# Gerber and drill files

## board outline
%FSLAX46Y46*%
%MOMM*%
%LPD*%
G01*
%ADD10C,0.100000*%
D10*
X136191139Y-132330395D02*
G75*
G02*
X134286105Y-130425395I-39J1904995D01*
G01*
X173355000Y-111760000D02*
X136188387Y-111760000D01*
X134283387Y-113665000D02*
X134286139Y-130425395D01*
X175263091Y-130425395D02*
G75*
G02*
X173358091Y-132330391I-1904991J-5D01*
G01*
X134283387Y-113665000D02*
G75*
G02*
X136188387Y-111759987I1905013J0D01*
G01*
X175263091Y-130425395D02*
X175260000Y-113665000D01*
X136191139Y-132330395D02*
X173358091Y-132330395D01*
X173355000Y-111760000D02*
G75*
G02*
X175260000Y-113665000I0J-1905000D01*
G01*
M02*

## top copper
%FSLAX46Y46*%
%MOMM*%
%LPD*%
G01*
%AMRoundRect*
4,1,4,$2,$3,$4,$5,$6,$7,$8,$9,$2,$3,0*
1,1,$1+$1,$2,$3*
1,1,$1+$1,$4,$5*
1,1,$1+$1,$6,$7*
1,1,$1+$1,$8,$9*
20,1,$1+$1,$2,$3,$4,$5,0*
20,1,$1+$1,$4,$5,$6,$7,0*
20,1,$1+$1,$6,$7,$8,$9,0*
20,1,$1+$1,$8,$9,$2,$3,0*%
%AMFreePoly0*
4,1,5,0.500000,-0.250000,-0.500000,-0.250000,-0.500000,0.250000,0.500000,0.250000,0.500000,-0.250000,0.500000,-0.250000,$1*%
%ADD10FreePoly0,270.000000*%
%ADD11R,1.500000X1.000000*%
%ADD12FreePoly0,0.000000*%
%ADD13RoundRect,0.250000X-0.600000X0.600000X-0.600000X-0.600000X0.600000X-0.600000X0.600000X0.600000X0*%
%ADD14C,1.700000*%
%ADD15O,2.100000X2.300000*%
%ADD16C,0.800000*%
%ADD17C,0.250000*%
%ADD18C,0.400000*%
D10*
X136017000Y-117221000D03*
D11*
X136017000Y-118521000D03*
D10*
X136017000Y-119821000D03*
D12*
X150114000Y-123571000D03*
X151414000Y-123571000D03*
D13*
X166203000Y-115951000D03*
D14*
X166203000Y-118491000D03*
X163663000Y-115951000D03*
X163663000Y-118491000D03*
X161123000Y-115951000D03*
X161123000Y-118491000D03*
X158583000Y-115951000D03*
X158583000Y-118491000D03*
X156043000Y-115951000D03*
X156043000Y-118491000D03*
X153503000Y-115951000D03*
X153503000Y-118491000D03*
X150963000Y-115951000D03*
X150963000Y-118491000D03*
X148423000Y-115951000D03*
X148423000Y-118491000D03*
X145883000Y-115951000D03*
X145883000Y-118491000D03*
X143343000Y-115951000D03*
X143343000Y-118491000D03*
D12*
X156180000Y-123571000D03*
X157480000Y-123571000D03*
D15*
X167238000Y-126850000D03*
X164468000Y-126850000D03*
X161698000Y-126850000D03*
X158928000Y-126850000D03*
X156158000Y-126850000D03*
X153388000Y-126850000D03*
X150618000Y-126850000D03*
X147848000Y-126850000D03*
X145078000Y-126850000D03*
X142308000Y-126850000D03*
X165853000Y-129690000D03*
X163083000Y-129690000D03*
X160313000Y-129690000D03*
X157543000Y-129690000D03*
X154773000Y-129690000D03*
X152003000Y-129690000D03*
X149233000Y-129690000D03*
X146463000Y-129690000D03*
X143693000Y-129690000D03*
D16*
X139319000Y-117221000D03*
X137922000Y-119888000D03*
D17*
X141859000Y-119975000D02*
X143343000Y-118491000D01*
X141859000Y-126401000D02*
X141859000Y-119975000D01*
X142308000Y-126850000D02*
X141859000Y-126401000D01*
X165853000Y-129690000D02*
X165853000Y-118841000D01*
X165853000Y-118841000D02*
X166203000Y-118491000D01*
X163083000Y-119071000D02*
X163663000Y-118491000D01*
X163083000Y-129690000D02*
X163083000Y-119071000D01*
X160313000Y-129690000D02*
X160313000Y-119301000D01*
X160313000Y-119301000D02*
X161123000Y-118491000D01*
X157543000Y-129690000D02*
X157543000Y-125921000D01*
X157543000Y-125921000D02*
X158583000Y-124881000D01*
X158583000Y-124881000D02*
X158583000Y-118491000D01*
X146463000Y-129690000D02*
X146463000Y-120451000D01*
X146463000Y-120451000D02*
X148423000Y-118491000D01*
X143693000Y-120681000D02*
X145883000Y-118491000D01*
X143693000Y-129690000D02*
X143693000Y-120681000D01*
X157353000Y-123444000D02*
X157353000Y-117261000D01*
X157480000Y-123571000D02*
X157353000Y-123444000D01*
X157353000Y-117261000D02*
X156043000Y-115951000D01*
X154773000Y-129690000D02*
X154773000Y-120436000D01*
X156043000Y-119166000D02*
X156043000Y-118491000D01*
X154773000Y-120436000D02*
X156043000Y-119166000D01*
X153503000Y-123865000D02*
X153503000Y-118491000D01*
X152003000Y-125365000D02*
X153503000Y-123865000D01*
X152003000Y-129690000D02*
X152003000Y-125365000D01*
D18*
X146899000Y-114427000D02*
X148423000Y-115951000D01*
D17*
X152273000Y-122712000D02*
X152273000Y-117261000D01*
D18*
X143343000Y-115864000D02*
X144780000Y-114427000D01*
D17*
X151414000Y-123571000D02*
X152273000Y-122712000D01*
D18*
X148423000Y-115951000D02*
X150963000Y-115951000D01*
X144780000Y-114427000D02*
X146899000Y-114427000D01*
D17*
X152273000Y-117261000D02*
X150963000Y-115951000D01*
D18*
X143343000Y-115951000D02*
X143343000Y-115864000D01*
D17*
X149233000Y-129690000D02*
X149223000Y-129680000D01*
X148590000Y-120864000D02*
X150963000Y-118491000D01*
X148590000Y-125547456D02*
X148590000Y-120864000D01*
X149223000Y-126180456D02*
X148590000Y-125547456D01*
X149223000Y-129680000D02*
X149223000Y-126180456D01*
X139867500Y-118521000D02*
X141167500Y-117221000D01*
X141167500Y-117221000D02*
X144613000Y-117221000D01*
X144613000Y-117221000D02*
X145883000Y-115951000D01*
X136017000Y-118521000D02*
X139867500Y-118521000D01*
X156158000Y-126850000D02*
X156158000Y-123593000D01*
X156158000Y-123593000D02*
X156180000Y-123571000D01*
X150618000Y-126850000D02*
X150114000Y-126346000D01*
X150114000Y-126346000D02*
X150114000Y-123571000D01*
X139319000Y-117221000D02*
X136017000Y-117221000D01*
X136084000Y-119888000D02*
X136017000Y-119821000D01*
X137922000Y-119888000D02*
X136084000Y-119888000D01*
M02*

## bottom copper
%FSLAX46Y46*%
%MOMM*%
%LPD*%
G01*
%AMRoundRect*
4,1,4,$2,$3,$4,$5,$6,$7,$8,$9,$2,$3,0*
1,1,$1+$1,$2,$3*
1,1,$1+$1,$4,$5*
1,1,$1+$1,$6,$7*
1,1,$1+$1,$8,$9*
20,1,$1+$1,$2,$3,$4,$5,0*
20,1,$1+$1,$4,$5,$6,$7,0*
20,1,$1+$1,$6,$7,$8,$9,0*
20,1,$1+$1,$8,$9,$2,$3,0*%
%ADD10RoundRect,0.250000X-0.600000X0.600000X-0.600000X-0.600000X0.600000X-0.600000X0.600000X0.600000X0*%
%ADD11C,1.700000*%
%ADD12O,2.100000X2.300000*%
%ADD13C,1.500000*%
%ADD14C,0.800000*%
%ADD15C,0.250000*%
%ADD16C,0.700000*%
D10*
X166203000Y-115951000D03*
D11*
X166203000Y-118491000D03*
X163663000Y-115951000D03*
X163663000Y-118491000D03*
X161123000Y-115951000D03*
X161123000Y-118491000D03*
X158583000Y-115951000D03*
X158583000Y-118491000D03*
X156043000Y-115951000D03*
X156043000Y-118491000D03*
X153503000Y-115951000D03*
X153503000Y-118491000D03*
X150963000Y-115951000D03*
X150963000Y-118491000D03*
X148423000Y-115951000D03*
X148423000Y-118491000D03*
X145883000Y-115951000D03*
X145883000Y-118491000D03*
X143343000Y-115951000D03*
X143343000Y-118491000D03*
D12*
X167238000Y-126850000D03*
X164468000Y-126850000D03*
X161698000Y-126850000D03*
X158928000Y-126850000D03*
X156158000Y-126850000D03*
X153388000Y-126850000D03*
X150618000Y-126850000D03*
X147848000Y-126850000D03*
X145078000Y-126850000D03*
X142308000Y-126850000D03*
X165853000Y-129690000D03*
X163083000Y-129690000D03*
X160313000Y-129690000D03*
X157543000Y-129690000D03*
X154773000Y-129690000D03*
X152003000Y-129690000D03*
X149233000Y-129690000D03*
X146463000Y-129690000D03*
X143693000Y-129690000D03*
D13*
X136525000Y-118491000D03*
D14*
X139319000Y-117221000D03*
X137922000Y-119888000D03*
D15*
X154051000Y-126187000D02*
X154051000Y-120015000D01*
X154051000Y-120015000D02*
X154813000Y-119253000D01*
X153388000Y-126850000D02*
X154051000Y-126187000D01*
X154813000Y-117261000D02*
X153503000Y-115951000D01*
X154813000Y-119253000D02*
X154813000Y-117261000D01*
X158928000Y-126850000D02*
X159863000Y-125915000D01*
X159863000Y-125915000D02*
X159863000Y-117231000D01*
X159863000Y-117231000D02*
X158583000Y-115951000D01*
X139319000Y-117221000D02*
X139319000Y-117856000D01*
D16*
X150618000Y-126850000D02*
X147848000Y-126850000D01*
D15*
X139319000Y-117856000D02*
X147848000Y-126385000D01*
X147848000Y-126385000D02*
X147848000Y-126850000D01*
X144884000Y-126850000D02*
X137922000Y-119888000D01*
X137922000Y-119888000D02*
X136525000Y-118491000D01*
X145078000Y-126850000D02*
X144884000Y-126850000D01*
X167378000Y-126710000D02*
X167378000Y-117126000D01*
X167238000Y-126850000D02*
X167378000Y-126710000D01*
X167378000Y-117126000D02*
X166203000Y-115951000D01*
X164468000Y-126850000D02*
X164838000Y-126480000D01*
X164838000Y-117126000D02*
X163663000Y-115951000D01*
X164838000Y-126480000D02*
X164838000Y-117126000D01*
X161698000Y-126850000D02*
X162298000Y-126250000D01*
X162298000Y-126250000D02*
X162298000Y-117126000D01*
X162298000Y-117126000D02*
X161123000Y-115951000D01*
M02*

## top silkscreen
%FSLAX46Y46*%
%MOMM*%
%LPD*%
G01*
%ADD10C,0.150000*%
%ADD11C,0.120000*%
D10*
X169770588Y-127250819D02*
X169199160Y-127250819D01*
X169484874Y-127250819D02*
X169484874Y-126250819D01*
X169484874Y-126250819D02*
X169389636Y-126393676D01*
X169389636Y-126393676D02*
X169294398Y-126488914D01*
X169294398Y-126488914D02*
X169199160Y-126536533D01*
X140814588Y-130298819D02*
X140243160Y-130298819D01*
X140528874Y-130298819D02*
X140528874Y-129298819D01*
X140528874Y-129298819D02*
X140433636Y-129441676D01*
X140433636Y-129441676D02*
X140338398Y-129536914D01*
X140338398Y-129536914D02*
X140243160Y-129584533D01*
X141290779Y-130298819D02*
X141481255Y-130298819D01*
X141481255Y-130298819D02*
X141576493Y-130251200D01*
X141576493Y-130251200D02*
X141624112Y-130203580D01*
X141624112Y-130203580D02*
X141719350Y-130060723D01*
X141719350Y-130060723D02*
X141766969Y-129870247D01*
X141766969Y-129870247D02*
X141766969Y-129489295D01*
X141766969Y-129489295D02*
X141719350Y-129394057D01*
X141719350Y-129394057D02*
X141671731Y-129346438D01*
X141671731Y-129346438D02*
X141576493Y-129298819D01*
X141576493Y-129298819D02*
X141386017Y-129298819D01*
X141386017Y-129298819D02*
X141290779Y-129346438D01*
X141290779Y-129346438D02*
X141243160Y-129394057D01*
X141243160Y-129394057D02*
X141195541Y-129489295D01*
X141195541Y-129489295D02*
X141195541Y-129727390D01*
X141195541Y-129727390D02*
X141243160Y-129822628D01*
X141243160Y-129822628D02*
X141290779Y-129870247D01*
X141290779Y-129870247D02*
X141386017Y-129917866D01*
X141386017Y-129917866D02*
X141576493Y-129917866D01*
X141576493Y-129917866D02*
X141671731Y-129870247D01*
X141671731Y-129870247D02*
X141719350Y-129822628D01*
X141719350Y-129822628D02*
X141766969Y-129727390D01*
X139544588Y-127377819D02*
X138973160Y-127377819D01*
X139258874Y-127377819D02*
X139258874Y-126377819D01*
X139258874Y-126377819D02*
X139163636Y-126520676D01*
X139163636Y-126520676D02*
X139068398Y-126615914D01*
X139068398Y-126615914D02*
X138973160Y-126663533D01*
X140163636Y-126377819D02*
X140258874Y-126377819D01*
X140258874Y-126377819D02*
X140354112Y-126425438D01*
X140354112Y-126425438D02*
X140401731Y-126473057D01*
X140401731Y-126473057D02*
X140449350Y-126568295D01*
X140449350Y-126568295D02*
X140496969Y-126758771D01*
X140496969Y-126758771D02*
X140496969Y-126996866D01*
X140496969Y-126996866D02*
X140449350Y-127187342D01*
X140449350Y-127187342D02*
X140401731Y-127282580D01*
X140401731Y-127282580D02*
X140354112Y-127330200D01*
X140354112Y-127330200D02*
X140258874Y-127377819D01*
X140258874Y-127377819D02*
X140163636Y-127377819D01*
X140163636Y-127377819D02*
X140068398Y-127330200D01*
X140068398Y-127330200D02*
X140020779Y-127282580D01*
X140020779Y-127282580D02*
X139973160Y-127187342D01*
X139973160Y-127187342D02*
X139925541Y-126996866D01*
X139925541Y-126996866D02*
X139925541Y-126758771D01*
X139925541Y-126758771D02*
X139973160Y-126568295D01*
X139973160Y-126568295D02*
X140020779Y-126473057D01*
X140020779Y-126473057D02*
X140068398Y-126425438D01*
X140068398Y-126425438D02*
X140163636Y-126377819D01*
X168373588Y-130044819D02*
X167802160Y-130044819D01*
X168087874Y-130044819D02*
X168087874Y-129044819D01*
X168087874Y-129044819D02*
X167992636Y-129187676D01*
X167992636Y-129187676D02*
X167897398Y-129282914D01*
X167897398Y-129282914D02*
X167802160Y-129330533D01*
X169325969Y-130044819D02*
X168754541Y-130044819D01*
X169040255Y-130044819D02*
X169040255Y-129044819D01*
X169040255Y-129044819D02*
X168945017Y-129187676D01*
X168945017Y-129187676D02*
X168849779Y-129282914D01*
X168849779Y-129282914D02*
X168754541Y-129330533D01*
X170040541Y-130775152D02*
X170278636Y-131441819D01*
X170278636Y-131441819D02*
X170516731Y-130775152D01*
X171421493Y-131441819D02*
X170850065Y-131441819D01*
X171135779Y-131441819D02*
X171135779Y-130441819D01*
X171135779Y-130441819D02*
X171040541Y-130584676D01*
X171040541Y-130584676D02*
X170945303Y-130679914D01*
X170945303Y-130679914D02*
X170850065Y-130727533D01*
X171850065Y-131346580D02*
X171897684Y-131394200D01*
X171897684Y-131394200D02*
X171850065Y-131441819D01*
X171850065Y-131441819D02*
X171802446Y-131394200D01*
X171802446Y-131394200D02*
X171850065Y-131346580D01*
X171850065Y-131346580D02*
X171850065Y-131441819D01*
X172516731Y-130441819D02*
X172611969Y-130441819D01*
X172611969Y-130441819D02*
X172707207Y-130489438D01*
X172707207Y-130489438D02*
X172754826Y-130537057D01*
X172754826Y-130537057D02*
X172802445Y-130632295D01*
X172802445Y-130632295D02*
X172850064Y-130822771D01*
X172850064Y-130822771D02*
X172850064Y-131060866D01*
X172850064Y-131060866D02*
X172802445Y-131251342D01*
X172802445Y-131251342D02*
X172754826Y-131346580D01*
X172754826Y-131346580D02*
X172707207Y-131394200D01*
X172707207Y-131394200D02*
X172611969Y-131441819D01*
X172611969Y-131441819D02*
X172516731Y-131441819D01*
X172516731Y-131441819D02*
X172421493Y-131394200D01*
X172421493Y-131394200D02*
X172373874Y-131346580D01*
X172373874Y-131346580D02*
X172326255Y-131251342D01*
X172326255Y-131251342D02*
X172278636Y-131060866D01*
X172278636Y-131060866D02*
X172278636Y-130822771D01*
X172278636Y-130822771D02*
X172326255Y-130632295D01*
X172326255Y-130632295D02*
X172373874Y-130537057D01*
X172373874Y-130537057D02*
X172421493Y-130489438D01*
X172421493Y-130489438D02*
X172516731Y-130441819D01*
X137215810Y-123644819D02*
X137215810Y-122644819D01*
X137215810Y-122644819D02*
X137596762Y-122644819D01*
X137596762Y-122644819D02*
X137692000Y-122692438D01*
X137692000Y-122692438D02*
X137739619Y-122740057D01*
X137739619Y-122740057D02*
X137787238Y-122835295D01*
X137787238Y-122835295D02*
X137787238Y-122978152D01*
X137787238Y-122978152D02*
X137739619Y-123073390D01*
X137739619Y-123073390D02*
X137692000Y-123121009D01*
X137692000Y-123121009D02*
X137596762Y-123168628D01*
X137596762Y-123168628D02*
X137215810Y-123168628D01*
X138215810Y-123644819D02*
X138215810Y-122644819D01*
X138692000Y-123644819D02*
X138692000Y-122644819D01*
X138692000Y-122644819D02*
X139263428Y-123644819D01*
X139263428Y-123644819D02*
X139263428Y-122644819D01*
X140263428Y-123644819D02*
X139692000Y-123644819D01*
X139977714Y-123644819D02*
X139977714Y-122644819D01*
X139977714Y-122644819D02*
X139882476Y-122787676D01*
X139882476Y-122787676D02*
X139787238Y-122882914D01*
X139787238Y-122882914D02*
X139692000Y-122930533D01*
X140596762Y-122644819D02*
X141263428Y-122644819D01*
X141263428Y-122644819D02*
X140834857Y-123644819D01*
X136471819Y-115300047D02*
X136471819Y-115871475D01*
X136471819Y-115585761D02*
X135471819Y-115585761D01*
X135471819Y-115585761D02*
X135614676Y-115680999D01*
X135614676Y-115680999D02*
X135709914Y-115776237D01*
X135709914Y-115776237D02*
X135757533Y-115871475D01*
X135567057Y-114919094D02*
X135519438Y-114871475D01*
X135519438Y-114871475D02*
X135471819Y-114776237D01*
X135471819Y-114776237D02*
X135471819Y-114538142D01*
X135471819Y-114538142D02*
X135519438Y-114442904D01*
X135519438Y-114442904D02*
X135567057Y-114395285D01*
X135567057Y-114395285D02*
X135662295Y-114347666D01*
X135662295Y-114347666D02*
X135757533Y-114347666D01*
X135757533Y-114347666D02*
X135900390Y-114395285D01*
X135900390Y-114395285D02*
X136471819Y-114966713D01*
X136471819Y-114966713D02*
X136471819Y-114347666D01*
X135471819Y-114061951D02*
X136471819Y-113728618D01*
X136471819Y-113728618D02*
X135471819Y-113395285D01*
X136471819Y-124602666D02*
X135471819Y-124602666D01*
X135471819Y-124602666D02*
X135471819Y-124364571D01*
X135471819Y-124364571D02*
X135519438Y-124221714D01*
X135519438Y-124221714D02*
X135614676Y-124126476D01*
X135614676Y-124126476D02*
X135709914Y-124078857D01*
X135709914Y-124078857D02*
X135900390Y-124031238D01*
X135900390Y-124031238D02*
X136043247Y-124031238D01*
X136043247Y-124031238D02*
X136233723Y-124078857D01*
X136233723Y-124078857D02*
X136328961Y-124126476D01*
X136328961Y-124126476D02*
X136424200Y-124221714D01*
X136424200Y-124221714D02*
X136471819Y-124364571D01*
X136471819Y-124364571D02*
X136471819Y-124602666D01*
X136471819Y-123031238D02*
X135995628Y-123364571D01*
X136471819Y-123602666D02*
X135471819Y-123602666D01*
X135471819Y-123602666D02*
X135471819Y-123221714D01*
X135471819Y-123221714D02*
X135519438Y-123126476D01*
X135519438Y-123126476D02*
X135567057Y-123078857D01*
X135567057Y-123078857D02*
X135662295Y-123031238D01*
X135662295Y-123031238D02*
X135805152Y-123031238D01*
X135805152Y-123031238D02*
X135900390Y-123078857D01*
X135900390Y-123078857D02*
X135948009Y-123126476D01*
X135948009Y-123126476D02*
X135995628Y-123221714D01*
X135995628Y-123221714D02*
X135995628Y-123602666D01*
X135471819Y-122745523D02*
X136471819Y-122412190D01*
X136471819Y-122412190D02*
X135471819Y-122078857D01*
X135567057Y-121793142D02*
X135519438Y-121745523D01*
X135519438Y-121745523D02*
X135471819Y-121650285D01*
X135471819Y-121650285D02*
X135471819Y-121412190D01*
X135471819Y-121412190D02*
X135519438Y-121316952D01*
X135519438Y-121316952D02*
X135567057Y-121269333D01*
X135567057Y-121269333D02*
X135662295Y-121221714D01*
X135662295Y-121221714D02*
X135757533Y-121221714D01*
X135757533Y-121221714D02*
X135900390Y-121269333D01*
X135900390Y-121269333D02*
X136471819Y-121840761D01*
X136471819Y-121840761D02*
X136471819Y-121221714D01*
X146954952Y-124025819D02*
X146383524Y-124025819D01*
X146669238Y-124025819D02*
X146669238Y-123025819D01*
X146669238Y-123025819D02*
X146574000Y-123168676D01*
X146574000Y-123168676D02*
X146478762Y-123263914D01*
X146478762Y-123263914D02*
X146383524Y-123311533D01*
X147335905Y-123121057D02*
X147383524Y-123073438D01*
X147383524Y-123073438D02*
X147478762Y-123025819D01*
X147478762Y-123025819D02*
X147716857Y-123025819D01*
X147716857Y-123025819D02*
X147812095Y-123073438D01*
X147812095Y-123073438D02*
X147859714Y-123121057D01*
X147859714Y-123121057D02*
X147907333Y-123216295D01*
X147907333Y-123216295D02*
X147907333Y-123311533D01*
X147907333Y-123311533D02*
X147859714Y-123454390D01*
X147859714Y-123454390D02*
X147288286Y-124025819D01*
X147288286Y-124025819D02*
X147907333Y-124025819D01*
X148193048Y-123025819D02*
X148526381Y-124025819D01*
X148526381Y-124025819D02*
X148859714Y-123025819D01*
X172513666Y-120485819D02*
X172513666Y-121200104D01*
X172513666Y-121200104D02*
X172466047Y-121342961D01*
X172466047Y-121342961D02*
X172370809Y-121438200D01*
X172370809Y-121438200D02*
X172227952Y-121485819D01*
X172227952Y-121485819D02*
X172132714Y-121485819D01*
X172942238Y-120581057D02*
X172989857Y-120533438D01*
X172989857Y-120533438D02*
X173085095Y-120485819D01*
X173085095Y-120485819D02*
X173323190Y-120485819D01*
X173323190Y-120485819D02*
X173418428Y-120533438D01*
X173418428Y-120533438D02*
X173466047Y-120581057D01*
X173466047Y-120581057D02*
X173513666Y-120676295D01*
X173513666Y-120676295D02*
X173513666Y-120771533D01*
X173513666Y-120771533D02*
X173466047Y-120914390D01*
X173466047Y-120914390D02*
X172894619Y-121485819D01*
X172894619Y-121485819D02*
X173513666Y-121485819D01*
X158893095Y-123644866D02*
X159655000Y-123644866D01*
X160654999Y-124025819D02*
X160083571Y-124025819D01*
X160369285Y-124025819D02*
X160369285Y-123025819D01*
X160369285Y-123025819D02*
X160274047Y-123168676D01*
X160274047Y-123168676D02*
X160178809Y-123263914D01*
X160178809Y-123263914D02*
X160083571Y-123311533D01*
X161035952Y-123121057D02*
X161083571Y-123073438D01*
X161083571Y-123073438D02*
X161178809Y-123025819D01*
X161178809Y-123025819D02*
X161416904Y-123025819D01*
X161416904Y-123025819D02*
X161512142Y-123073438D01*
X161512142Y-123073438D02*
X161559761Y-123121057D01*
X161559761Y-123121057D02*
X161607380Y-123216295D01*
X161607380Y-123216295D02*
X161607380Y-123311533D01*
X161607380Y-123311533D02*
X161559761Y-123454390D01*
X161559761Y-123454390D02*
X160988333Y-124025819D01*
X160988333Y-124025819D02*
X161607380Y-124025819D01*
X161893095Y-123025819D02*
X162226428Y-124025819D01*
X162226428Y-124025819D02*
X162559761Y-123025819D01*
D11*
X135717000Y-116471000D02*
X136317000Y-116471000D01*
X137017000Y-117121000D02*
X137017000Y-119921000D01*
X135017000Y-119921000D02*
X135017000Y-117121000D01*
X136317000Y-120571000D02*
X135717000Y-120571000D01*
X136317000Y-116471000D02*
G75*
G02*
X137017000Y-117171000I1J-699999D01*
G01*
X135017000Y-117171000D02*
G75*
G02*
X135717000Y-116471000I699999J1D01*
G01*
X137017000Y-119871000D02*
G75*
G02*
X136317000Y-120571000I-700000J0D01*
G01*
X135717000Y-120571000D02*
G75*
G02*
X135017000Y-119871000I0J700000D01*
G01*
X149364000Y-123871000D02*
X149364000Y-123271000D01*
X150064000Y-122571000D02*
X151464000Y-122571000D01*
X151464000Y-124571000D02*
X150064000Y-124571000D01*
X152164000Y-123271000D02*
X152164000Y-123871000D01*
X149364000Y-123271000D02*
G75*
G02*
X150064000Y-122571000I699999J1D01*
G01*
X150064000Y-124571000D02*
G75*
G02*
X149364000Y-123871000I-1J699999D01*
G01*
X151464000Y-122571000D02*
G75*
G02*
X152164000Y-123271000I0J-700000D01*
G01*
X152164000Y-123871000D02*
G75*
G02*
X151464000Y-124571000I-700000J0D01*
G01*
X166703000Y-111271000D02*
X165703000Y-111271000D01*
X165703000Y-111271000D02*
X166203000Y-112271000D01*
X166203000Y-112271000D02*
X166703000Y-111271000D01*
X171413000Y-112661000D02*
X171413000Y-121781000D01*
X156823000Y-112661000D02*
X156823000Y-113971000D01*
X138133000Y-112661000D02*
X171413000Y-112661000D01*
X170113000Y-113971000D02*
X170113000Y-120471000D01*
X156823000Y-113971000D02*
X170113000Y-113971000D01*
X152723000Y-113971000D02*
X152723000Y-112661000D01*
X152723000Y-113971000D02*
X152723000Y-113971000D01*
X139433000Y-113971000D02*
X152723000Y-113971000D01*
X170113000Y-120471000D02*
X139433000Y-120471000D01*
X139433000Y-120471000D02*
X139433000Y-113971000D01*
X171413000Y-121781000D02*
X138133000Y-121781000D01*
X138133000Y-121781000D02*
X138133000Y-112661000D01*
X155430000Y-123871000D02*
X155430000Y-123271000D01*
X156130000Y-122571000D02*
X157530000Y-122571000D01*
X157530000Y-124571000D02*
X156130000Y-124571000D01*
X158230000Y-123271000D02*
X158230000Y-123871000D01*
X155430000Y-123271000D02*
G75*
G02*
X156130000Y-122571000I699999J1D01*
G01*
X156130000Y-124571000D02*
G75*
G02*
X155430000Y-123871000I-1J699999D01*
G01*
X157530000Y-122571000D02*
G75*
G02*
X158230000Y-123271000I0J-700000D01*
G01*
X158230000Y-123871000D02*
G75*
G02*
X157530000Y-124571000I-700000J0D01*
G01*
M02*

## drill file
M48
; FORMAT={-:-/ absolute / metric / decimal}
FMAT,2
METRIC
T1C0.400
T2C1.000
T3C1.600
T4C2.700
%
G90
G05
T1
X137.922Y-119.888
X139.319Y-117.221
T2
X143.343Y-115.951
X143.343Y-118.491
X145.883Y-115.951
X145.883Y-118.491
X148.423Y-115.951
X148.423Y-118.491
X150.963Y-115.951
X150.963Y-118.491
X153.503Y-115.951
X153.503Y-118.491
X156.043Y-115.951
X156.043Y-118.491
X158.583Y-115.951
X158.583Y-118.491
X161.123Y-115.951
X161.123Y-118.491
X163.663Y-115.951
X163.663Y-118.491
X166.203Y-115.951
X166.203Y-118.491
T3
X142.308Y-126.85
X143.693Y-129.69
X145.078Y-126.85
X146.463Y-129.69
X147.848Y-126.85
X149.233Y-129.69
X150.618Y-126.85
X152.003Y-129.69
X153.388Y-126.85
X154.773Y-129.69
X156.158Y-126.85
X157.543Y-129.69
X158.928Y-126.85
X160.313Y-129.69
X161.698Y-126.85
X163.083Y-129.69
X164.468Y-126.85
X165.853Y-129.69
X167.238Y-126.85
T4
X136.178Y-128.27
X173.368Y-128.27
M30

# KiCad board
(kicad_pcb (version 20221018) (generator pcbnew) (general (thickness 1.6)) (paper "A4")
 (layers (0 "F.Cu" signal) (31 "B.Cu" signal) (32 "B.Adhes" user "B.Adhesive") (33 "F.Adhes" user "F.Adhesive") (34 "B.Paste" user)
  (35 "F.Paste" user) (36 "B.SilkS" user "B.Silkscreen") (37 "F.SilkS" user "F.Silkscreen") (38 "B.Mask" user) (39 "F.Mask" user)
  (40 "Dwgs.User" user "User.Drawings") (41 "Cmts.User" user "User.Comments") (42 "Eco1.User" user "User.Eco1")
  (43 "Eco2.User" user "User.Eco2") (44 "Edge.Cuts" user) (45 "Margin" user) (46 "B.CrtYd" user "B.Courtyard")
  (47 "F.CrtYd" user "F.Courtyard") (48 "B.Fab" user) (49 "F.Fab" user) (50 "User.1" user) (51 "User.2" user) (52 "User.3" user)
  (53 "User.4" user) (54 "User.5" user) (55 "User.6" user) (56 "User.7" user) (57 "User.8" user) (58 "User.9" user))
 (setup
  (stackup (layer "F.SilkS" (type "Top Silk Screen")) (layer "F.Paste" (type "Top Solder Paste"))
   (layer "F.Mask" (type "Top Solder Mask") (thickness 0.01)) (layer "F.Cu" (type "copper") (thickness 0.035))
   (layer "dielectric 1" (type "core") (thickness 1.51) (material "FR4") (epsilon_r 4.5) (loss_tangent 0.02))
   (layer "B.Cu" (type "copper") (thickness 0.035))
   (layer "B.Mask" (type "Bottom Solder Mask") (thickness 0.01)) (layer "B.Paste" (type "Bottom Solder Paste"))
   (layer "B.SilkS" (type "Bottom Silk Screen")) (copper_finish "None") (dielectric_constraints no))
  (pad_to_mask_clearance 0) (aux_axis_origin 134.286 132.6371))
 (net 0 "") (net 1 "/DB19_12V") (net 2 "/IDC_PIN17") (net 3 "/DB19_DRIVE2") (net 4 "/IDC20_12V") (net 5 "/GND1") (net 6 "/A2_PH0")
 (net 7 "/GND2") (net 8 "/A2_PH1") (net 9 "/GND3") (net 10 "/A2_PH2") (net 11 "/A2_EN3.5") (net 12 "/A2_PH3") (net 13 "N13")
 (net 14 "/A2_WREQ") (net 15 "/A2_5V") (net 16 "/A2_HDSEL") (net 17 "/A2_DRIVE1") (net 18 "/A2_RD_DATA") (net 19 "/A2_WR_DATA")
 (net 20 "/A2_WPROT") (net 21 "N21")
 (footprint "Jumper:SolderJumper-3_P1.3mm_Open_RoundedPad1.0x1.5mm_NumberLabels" (layer "F.Cu") (at 136.017 118.521 -90)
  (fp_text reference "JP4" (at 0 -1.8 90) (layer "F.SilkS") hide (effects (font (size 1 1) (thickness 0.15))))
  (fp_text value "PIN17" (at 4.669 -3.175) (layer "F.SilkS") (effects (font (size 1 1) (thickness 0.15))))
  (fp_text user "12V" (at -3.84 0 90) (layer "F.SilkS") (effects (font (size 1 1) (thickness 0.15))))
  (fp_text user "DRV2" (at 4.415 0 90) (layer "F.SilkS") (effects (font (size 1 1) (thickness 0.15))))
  (fp_line (start -2.05 0.3) (end -2.05 -0.3) (stroke (width 0.12) (type solid)) (layer "F.SilkS"))
  (fp_line (start -1.4 -1) (end 1.4 -1) (stroke (width 0.12) (type solid)) (layer "F.SilkS"))
  (fp_line (start 1.4 1) (end -1.4 1) (stroke (width 0.12) (type solid)) (layer "F.SilkS"))
  (fp_line (start 2.05 -0.3) (end 2.05 0.3) (stroke (width 0.12) (type solid)) (layer "F.SilkS"))
  (fp_arc (start -2.05 -0.3) (mid -1.844975 -0.794975) (end -1.35 -1) (stroke (width 0.12) (type solid)) (layer "F.SilkS"))
  (fp_arc (start -1.35 1) (mid -1.844975 0.794975) (end -2.05 0.3) (stroke (width 0.12) (type solid)) (layer "F.SilkS"))
  (fp_arc (start 1.35 -1) (mid 1.844975 -0.794975) (end 2.05 -0.3) (stroke (width 0.12) (type solid)) (layer "F.SilkS"))
  (fp_arc (start 2.05 0.3) (mid 1.844975 0.794975) (end 1.35 1) (stroke (width 0.12) (type solid)) (layer "F.SilkS"))
  (pad "1" smd custom (at -1.3 0 270) (size 1 0.5) (layers "F.Cu" "F.Mask") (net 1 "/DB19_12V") (zone_connect 2)
   (options (clearance outline) (anchor rect)) (primitives))
  (pad "2" smd rect (at 0 0 270) (size 1 1.5) (layers "F.Cu" "F.Mask") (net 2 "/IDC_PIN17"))
  (pad "3" smd custom (at 1.3 0 270) (size 1 0.5) (layers "F.Cu" "F.Mask") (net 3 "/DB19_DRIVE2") (zone_connect 2)
   (options (clearance outline) (anchor rect)) (primitives)))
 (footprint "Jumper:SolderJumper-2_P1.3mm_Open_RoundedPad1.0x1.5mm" (layer "F.Cu") (at 150.764 123.571)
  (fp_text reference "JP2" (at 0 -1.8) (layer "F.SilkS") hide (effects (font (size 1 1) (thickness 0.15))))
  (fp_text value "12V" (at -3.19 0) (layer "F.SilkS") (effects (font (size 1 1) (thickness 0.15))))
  (fp_line (start -1.4 0.3) (end -1.4 -0.3) (stroke (width 0.12) (type solid)) (layer "F.SilkS"))
  (fp_line (start -0.7 -1) (end 0.7 -1) (stroke (width 0.12) (type solid)) (layer "F.SilkS"))
  (fp_line (start 0.7 1) (end -0.7 1) (stroke (width 0.12) (type solid)) (layer "F.SilkS"))
  (fp_line (start 1.4 -0.3) (end 1.4 0.3) (stroke (width 0.12) (type solid)) (layer "F.SilkS"))
  (fp_arc (start -1.4 -0.3) (mid -1.194975 -0.794975) (end -0.7 -1) (stroke (width 0.12) (type solid)) (layer "F.SilkS"))
  (fp_arc (start -0.7 1) (mid -1.194975 0.794975) (end -1.4 0.3) (stroke (width 0.12) (type solid)) (layer "F.SilkS"))
  (fp_arc (start 0.7 -1) (mid 1.194975 -0.794975) (end 1.4 -0.3) (stroke (width 0.12) (type solid)) (layer "F.SilkS"))
  (fp_arc (start 1.4 0.3) (mid 1.194975 0.794975) (end 0.7 1) (stroke (width 0.12) (type solid)) (layer "F.SilkS"))
  (pad "1" smd custom (at -0.65 0) (size 1 0.5) (layers "F.Cu" "F.Mask") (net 1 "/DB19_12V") (zone_connect 2)
   (options (clearance outline) (anchor rect)) (primitives))
  (pad "2" smd custom (at 0.65 0) (size 1 0.5) (layers "F.Cu" "F.Mask") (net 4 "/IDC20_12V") (zone_connect 2)
   (options (clearance outline) (anchor rect)) (primitives)))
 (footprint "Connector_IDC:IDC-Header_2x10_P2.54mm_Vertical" (layer "F.Cu") (at 166.203 115.951 -90)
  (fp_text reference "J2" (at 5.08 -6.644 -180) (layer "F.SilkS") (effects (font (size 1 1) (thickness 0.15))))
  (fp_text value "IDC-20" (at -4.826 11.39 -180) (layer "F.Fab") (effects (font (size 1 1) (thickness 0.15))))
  (fp_line (start -4.68 -0.5) (end -4.68 0.5) (stroke (width 0.12) (type solid)) (layer "F.SilkS"))
  (fp_line (start -4.68 0.5) (end -3.68 0) (stroke (width 0.12) (type solid)) (layer "F.SilkS"))
  (fp_line (start -3.68 0) (end -4.68 -0.5) (stroke (width 0.12) (type solid)) (layer "F.SilkS"))
  (fp_line (start -3.29 -5.21) (end 5.83 -5.21) (stroke (width 0.12) (type solid)) (layer "F.SilkS"))
  (fp_line (start -3.29 9.38) (end -1.98 9.38) (stroke (width 0.12) (type solid)) (layer "F.SilkS"))
  (fp_line (start -3.29 28.07) (end -3.29 -5.21) (stroke (width 0.12) (type solid)) (layer "F.SilkS"))
  (fp_line (start -1.98 -3.91) (end 4.52 -3.91) (stroke (width 0.12) (type solid)) (layer "F.SilkS"))
  (fp_line (start -1.98 9.38) (end -1.98 -3.91) (stroke (width 0.12) (type solid)) (layer "F.SilkS"))
  (fp_line (start -1.98 13.48) (end -3.29 13.48) (stroke (width 0.12) (type solid)) (layer "F.SilkS"))
  (fp_line (start -1.98 13.48) (end -1.98 13.48) (stroke (width 0.12) (type solid)) (layer "F.SilkS"))
  (fp_line (start -1.98 26.77) (end -1.98 13.48) (stroke (width 0.12) (type solid)) (layer "F.SilkS"))
  (fp_line (start 4.52 -3.91) (end 4.52 26.77) (stroke (width 0.12) (type solid)) (layer "F.SilkS"))
  (fp_line (start 4.52 26.77) (end -1.98 26.77) (stroke (width 0.12) (type solid)) (layer "F.SilkS"))
  (fp_line (start 5.83 -5.21) (end 5.83 28.07) (stroke (width 0.12) (type solid)) (layer "F.SilkS"))
  (fp_line (start 5.83 28.07) (end -3.29 28.07) (stroke (width 0.12) (type solid)) (layer "F.SilkS"))
  (pad "1" thru_hole roundrect (at 0 0 270) (size 1.7 1.7) (drill 1) (layers "*.Cu" "*.Mask") (roundrect_rratio 0.1470588235)
   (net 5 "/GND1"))
  (pad "2" thru_hole circle (at 2.54 0 270) (size 1.7 1.7) (drill 1) (layers "*.Cu" "*.Mask") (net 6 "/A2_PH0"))
  (pad "3" thru_hole circle (at 0 2.54 270) (size 1.7 1.7) (drill 1) (layers "*.Cu" "*.Mask") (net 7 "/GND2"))
  (pad "4" thru_hole circle (at 2.54 2.54 270) (size 1.7 1.7) (drill 1) (layers "*.Cu" "*.Mask") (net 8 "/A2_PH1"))
  (pad "5" thru_hole circle (at 0 5.08 270) (size 1.7 1.7) (drill 1) (layers "*.Cu" "*.Mask") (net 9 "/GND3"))
  (pad "6" thru_hole circle (at 2.54 5.08 270) (size 1.7 1.7) (drill 1) (layers "*.Cu" "*.Mask") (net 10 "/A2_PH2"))
  (pad "7" thru_hole circle (at 0 7.62 270) (size 1.7 1.7) (drill 1) (layers "*.Cu" "*.Mask") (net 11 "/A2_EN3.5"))
  (pad "8" thru_hole circle (at 2.54 7.62 270) (size 1.7 1.7) (drill 1) (layers "*.Cu" "*.Mask") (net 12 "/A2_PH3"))
  (pad "9" thru_hole circle (at 0 10.16 270) (size 1.7 1.7) (drill 1) (layers "*.Cu" "*.Mask") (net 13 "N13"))
  (pad "10" thru_hole circle (at 2.54 10.16 270) (size 1.7 1.7) (drill 1) (layers "*.Cu" "*.Mask") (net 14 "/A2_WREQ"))
  (pad "11" thru_hole circle (at 0 12.7 270) (size 1.7 1.7) (drill 1) (layers "*.Cu" "*.Mask") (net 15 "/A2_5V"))
  (pad "12" thru_hole circle (at 2.54 12.7 270) (size 1.7 1.7) (drill 1) (layers "*.Cu" "*.Mask") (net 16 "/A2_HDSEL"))
  (pad "13" thru_hole circle (at 0 15.24 270) (size 1.7 1.7) (drill 1) (layers "*.Cu" "*.Mask") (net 4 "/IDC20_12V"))
  (pad "14" thru_hole circle (at 2.54 15.24 270) (size 1.7 1.7) (drill 1) (layers "*.Cu" "*.Mask") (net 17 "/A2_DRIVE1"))
  (pad "15" thru_hole circle (at 0 17.78 270) (size 1.7 1.7) (drill 1) (layers "*.Cu" "*.Mask") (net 4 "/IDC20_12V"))
  (pad "16" thru_hole circle (at 2.54 17.78 270) (size 1.7 1.7) (drill 1) (layers "*.Cu" "*.Mask") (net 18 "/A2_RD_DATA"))
  (pad "17" thru_hole circle (at 0 20.32 270) (size 1.7 1.7) (drill 1) (layers "*.Cu" "*.Mask") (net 2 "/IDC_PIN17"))
  (pad "18" thru_hole circle (at 2.54 20.32 270) (size 1.7 1.7) (drill 1) (layers "*.Cu" "*.Mask") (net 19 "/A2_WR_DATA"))
  (pad "19" thru_hole circle (at 0 22.86 270) (size 1.7 1.7) (drill 1) (layers "*.Cu" "*.Mask") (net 4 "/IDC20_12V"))
  (pad "20" thru_hole circle (at 2.54 22.86 270) (size 1.7 1.7) (drill 1) (layers "*.Cu" "*.Mask") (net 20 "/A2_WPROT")))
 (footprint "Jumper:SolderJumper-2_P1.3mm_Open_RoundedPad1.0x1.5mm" (layer "F.Cu") (at 156.83 123.571)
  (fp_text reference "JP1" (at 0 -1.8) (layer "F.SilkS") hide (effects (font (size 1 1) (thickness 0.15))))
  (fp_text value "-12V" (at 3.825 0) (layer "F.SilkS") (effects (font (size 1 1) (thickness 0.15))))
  (fp_line (start -1.4 0.3) (end -1.4 -0.3) (stroke (width 0.12) (type solid)) (layer "F.SilkS"))
  (fp_line (start -0.7 -1) (end 0.7 -1) (stroke (width 0.12) (type solid)) (layer "F.SilkS"))
  (fp_line (start 0.7 1) (end -0.7 1) (stroke (width 0.12) (type solid)) (layer "F.SilkS"))
  (fp_line (start 1.4 -0.3) (end 1.4 0.3) (stroke (width 0.12) (type solid)) (layer "F.SilkS"))
  (fp_arc (start -1.4 -0.3) (mid -1.194975 -0.794975) (end -0.7 -1) (stroke (width 0.12) (type solid)) (layer "F.SilkS"))
  (fp_arc (start -0.7 1) (mid -1.194975 0.794975) (end -1.4 0.3) (stroke (width 0.12) (type solid)) (layer "F.SilkS"))
  (fp_arc (start 0.7 -1) (mid 1.194975 -0.794975) (end 1.4 -0.3) (stroke (width 0.12) (type solid)) (layer "F.SilkS"))
  (fp_arc (start 1.4 0.3) (mid 1.194975 0.794975) (end 0.7 1) (stroke (width 0.12) (type solid)) (layer "F.SilkS"))
  (pad "1" smd custom (at -0.65 0) (size 1 0.5) (layers "F.Cu" "F.Mask") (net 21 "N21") (zone_connect 2)
   (options (clearance outline) (anchor rect)) (primitives))
  (pad "2" smd custom (at 0.65 0) (size 1 0.5) (layers "F.Cu" "F.Mask") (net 13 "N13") (zone_connect 2)
   (options (clearance outline) (anchor rect)) (primitives)))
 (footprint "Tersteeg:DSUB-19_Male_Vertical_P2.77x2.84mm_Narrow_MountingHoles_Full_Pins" (layer "B.Cu") (at 167.238 126.85 180)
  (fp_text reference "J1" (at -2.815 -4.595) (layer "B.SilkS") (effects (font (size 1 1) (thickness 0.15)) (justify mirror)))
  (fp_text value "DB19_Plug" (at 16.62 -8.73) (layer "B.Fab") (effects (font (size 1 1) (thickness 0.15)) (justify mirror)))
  (pad "" np_thru_hole circle (at -6.13 -1.42 180) (size 2.7 2.7) (drill 2.7) (layers "F&B.Cu" "*.Mask"))
  (pad "" np_thru_hole circle (at 31.06 -1.42 180) (size 2.7 2.7) (drill 2.7) (layers "F&B.Cu" "*.Mask"))
  (pad "1" thru_hole oval (at 0 0 180) (size 2.1 2.3) (drill 1.6) (layers "*.Cu" "*.Mask") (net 5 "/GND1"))
  (pad "2" thru_hole oval (at 2.77 0 180) (size 2.1 2.3) (drill 1.6) (layers "*.Cu" "*.Mask") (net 7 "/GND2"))
  (pad "3" thru_hole oval (at 5.54 0 180) (size 2.1 2.3) (drill 1.6) (layers "*.Cu" "*.Mask") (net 9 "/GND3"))
  (pad "4" thru_hole oval (at 8.31 0 180) (size 2.1 2.3) (drill 1.6) (layers "*.Cu" "*.Mask") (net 11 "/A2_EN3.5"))
  (pad "5" thru_hole oval (at 11.08 0 180) (size 2.1 2.3) (drill 1.6) (layers "*.Cu" "*.Mask") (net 21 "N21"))
  (pad "6" thru_hole oval (at 13.85 0 180) (size 2.1 2.3) (drill 1.6) (layers "*.Cu" "*.Mask") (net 15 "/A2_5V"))
  (pad "7" thru_hole oval (at 16.62 0 180) (size 2.1 2.3) (drill 1.6) (layers "*.Cu" "*.Mask") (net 1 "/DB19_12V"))
  (pad "8" thru_hole oval (at 19.39 0 180) (size 2.1 2.3) (drill 1.6) (layers "*.Cu" "*.Mask") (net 1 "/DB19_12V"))
  (pad "9" thru_hole oval (at 22.16 0 180) (size 2.1 2.3) (drill 1.6) (layers "*.Cu" "*.Mask") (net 3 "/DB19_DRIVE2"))
  (pad "10" thru_hole oval (at 24.93 0 180) (size 2.1 2.3) (drill 1.6) (layers "*.Cu" "*.Mask") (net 20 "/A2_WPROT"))
  (pad "11" thru_hole oval (at 1.385 -2.84 180) (size 2.1 2.3) (drill 1.6) (layers "*.Cu" "*.Mask") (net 6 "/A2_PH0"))
  (pad "12" thru_hole oval (at 4.155 -2.84 180) (size 2.1 2.3) (drill 1.6) (layers "*.Cu" "*.Mask") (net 8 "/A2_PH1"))
  (pad "13" thru_hole oval (at 6.925 -2.84 180) (size 2.1 2.3) (drill 1.6) (layers "*.Cu" "*.Mask") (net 10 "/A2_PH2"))
  (pad "14" thru_hole oval (at 9.695 -2.84 180) (size 2.1 2.3) (drill 1.6) (layers "*.Cu" "*.Mask") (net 12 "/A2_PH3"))
  (pad "15" thru_hole oval (at 12.465 -2.84 180) (size 2.1 2.3) (drill 1.6) (layers "*.Cu" "*.Mask") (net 14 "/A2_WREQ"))
  (pad "16" thru_hole oval (at 15.235 -2.84 180) (size 2.1 2.3) (drill 1.6) (layers "*.Cu" "*.Mask") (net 16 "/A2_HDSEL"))
  (pad "17" thru_hole oval (at 18.005 -2.84 180) (size 2.1 2.3) (drill 1.6) (layers "*.Cu" "*.Mask") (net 17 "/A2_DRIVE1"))
  (pad "18" thru_hole oval (at 20.775 -2.84 180) (size 2.1 2.3) (drill 1.6) (layers "*.Cu" "*.Mask") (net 18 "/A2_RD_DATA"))
  (pad "19" thru_hole oval (at 23.545 -2.84 180) (size 2.1 2.3) (drill 1.6) (layers "*.Cu" "*.Mask") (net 19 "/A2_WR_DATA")))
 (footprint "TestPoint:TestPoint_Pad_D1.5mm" (layer "B.Cu") (at 136.525 118.491 180)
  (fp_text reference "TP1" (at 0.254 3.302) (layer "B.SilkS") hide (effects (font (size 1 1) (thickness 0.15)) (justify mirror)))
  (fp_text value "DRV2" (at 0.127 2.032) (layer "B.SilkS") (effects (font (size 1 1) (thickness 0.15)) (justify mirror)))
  (pad "1" smd circle (at 0 0 180) (size 1.5 1.5) (layers "B.Cu" "B.Mask") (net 3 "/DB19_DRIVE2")))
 (gr_arc (start 136.191139 132.330395) (mid 134.844101 131.772433) (end 134.286139 130.425395) (stroke (width 0.1) (type default))
  (layer "Edge.Cuts"))
 (gr_line (start 173.355 111.76) (end 136.188387 111.76) (stroke (width 0.1) (type default)) (layer "Edge.Cuts"))
 (gr_line (start 134.283387 113.665) (end 134.286139 130.425395) (stroke (width 0.1) (type default)) (layer "Edge.Cuts"))
 (gr_arc (start 175.263091 130.425395) (mid 174.705129 131.772433) (end 173.358091 132.330395) (stroke (width 0.1) (type default))
  (layer "Edge.Cuts"))
 (gr_arc (start 134.283387 113.665) (mid 134.841349 112.317962) (end 136.188387 111.76) (stroke (width 0.1) (type default))
  (layer "Edge.Cuts"))
 (gr_line (start 175.263091 130.425395) (end 175.26 113.665) (stroke (width 0.1) (type default)) (layer "Edge.Cuts"))
 (gr_line locked (start 136.191139 132.330395) (end 173.358091 132.330395) (stroke (width 0.1) (type default)) (layer "Edge.Cuts"))
 (gr_arc (start 173.355 111.76) (mid 174.702038 112.317962) (end 175.26 113.665) (stroke (width 0.1) (type default)) (layer "Edge.Cuts"))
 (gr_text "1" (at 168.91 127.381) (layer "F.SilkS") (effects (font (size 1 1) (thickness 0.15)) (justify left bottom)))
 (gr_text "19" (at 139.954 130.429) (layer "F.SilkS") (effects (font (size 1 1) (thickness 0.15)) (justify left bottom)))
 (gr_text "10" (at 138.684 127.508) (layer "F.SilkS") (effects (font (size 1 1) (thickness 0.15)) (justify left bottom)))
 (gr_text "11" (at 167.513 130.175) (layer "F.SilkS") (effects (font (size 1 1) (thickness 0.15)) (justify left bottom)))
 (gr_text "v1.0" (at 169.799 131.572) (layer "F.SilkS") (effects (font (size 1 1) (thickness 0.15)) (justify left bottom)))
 (segment (start 154.051 126.187) (end 154.051 120.015) (width 0.25) (layer "B.Cu") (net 15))
 (segment (start 154.051 120.015) (end 154.813 119.253) (width 0.25) (layer "B.Cu") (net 15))
 (segment (start 153.388 126.85) (end 154.051 126.187) (width 0.25) (layer "B.Cu") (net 15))
 (segment (start 154.813 117.261) (end 153.503 115.951) (width 0.25) (layer "B.Cu") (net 15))
 (segment (start 154.813 119.253) (end 154.813 117.261) (width 0.25) (layer "B.Cu") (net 15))
 (segment (start 141.859 119.975) (end 143.343 118.491) (width 0.25) (layer "F.Cu") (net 20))
 (segment (start 141.859 126.401) (end 141.859 119.975) (width 0.25) (layer "F.Cu") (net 20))
 (segment (start 142.308 126.85) (end 141.859 126.401) (width 0.25) (layer "F.Cu") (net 20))
 (segment (start 165.853 129.69) (end 165.853 118.841) (width 0.25) (layer "F.Cu") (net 6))
 (segment (start 165.853 118.841) (end 166.203 118.491) (width 0.25) (layer "F.Cu") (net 6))
 (segment (start 163.083 119.071) (end 163.663 118.491) (width 0.25) (layer "F.Cu") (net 8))
 (segment (start 163.083 129.69) (end 163.083 119.071) (width 0.25) (layer "F.Cu") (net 8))
 (segment (start 160.313 129.69) (end 160.313 119.301) (width 0.25) (layer "F.Cu") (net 10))
 (segment (start 160.313 119.301) (end 161.123 118.491) (width 0.25) (layer "F.Cu") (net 10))
 (segment (start 157.543 129.69) (end 157.543 125.921) (width 0.25) (layer "F.Cu") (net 12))
 (segment (start 157.543 125.921) (end 158.583 124.881) (width 0.25) (layer "F.Cu") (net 12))
 (segment (start 158.583 124.881) (end 158.583 118.491) (width 0.25) (layer "F.Cu") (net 12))
 (segment (start 146.463 129.69) (end 146.463 120.451) (width 0.25) (layer "F.Cu") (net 18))
 (segment (start 146.463 120.451) (end 148.423 118.491) (width 0.25) (layer "F.Cu") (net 18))
 (segment (start 143.693 120.681) (end 145.883 118.491) (width 0.25) (layer "F.Cu") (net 19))
 (segment (start 143.693 129.69) (end 143.693 120.681) (width 0.25) (layer "F.Cu") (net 19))
 (segment (start 158.928 126.85) (end 159.863 125.915) (width 0.25) (layer "B.Cu") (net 11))
 (segment (start 159.863 125.915) (end 159.863 117.231) (width 0.25) (layer "B.Cu") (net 11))
 (segment (start 159.863 117.231) (end 158.583 115.951) (width 0.25) (layer "B.Cu") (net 11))
 (segment (start 157.353 123.444) (end 157.353 117.261) (width 0.25) (layer "F.Cu") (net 13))
 (segment (start 157.48 123.571) (end 157.353 123.444) (width 0.25) (layer "F.Cu") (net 13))
 (segment (start 157.353 117.261) (end 156.043 115.951) (width 0.25) (layer "F.Cu") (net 13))
 (segment (start 154.773 129.69) (end 154.773 120.436) (width 0.25) (layer "F.Cu") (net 14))
 (segment (start 156.043 119.166) (end 156.043 118.491) (width 0.25) (layer "F.Cu") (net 14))
 (segment (start 154.773 120.436) (end 156.043 119.166) (width 0.25) (layer "F.Cu") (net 14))
 (segment (start 153.503 123.865) (end 153.503 118.491) (width 0.25) (layer "F.Cu") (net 16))
 (segment (start 152.003 125.365) (end 153.503 123.865) (width 0.25) (layer "F.Cu") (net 16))
 (segment (start 152.003 129.69) (end 152.003 125.365) (width 0.25) (layer "F.Cu") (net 16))
 (segment (start 146.899 114.427) (end 148.423 115.951) (width 0.4) (layer "F.Cu") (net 4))
 (segment (start 152.273 122.712) (end 152.273 117.261) (width 0.25) (layer "F.Cu") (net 4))
 (segment (start 143.343 115.864) (end 144.78 114.427) (width 0.4) (layer "F.Cu") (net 4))
 (segment (start 151.414 123.571) (end 152.273 122.712) (width 0.25) (layer "F.Cu") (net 4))
 (segment (start 148.423 115.951) (end 150.963 115.951) (width 0.4) (layer "F.Cu") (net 4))
 (segment (start 144.78 114.427) (end 146.899 114.427) (width 0.4) (layer "F.Cu") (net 4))
 (segment (start 152.273 117.261) (end 150.963 115.951) (width 0.25) (layer "F.Cu") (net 4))
 (segment (start 143.343 115.951) (end 143.343 115.864) (width 0.4) (layer "F.Cu") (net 4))
 (segment (start 149.233 129.69) (end 149.223 129.68) (width 0.25) (layer "F.Cu") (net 17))
 (segment (start 148.59 120.864) (end 150.963 118.491) (width 0.25) (layer "F.Cu") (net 17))
 (segment (start 148.59 125.547456) (end 148.59 120.864) (width 0.25) (layer "F.Cu") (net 17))
 (segment (start 149.223 126.180456) (end 148.59 125.547456) (width 0.25) (layer "F.Cu") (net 17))
 (segment (start 149.223 129.68) (end 149.223 126.180456) (width 0.25) (layer "F.Cu") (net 17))
 (segment (start 139.8675 118.521) (end 141.1675 117.221) (width 0.25) (layer "F.Cu") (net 2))
 (segment (start 141.1675 117.221) (end 144.613 117.221) (width 0.25) (layer "F.Cu") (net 2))
 (segment (start 144.613 117.221) (end 145.883 115.951) (width 0.25) (layer "F.Cu") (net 2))
 (segment (start 136.017 118.521) (end 139.8675 118.521) (width 0.25) (layer "F.Cu") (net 2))
 (segment (start 156.158 126.85) (end 156.158 123.593) (width 0.25) (layer "F.Cu") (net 21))
 (segment (start 156.158 123.593) (end 156.18 123.571) (width 0.25) (layer "F.Cu") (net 21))
 (segment (start 150.618 126.85) (end 150.114 126.346) (width 0.25) (layer "F.Cu") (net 1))
 (segment (start 150.114 126.346) (end 150.114 123.571) (width 0.25) (layer "F.Cu") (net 1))
 (segment (start 139.319 117.221) (end 136.017 117.221) (width 0.25) (layer "F.Cu") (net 1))
 (via (at 139.319 117.221) (size 0.8) (drill 0.4) (layers "F.Cu" "B.Cu") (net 1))
 (segment (start 139.319 117.221) (end 139.319 117.856) (width 0.25) (layer "B.Cu") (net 1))
 (segment (start 150.618 126.85) (end 147.848 126.85) (width 0.7) (layer "B.Cu") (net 1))
 (segment (start 139.319 117.856) (end 147.848 126.385) (width 0.25) (layer "B.Cu") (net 1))
 (segment (start 147.848 126.385) (end 147.848 126.85) (width 0.25) (layer "B.Cu") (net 1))
 (segment (start 136.084 119.888) (end 136.017 119.821) (width 0.25) (layer "F.Cu") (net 3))
 (segment (start 137.922 119.888) (end 136.084 119.888) (width 0.25) (layer "F.Cu") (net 3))
 (via (at 137.922 119.888) (size 0.8) (drill 0.4) (layers "F.Cu" "B.Cu") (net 3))
 (segment (start 144.884 126.85) (end 137.922 119.888) (width 0.25) (layer "B.Cu") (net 3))
 (segment (start 137.922 119.888) (end 136.525 118.491) (width 0.25) (layer "B.Cu") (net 3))
 (segment (start 145.078 126.85) (end 144.884 126.85) (width 0.25) (layer "B.Cu") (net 3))
 (segment (start 167.378 126.71) (end 167.378 117.126) (width 0.25) (layer "B.Cu") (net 5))
 (segment (start 167.238 126.85) (end 167.378 126.71) (width 0.25) (layer "B.Cu") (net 5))
 (segment (start 167.378 117.126) (end 166.203 115.951) (width 0.25) (layer "B.Cu") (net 5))
 (segment (start 164.468 126.85) (end 164.838 126.48) (width 0.25) (layer "B.Cu") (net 7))
 (segment (start 164.838 117.126) (end 163.663 115.951) (width 0.25) (layer "B.Cu") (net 7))
 (segment (start 164.838 126.48) (end 164.838 117.126) (width 0.25) (layer "B.Cu") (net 7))
 (segment (start 161.698 126.85) (end 162.298 126.25) (width 0.25) (layer "B.Cu") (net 9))
 (segment (start 162.298 126.25) (end 162.298 117.126) (width 0.25) (layer "B.Cu") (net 9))
 (segment (start 162.298 117.126) (end 161.123 115.951) (width 0.25) (layer "B.Cu") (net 9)))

